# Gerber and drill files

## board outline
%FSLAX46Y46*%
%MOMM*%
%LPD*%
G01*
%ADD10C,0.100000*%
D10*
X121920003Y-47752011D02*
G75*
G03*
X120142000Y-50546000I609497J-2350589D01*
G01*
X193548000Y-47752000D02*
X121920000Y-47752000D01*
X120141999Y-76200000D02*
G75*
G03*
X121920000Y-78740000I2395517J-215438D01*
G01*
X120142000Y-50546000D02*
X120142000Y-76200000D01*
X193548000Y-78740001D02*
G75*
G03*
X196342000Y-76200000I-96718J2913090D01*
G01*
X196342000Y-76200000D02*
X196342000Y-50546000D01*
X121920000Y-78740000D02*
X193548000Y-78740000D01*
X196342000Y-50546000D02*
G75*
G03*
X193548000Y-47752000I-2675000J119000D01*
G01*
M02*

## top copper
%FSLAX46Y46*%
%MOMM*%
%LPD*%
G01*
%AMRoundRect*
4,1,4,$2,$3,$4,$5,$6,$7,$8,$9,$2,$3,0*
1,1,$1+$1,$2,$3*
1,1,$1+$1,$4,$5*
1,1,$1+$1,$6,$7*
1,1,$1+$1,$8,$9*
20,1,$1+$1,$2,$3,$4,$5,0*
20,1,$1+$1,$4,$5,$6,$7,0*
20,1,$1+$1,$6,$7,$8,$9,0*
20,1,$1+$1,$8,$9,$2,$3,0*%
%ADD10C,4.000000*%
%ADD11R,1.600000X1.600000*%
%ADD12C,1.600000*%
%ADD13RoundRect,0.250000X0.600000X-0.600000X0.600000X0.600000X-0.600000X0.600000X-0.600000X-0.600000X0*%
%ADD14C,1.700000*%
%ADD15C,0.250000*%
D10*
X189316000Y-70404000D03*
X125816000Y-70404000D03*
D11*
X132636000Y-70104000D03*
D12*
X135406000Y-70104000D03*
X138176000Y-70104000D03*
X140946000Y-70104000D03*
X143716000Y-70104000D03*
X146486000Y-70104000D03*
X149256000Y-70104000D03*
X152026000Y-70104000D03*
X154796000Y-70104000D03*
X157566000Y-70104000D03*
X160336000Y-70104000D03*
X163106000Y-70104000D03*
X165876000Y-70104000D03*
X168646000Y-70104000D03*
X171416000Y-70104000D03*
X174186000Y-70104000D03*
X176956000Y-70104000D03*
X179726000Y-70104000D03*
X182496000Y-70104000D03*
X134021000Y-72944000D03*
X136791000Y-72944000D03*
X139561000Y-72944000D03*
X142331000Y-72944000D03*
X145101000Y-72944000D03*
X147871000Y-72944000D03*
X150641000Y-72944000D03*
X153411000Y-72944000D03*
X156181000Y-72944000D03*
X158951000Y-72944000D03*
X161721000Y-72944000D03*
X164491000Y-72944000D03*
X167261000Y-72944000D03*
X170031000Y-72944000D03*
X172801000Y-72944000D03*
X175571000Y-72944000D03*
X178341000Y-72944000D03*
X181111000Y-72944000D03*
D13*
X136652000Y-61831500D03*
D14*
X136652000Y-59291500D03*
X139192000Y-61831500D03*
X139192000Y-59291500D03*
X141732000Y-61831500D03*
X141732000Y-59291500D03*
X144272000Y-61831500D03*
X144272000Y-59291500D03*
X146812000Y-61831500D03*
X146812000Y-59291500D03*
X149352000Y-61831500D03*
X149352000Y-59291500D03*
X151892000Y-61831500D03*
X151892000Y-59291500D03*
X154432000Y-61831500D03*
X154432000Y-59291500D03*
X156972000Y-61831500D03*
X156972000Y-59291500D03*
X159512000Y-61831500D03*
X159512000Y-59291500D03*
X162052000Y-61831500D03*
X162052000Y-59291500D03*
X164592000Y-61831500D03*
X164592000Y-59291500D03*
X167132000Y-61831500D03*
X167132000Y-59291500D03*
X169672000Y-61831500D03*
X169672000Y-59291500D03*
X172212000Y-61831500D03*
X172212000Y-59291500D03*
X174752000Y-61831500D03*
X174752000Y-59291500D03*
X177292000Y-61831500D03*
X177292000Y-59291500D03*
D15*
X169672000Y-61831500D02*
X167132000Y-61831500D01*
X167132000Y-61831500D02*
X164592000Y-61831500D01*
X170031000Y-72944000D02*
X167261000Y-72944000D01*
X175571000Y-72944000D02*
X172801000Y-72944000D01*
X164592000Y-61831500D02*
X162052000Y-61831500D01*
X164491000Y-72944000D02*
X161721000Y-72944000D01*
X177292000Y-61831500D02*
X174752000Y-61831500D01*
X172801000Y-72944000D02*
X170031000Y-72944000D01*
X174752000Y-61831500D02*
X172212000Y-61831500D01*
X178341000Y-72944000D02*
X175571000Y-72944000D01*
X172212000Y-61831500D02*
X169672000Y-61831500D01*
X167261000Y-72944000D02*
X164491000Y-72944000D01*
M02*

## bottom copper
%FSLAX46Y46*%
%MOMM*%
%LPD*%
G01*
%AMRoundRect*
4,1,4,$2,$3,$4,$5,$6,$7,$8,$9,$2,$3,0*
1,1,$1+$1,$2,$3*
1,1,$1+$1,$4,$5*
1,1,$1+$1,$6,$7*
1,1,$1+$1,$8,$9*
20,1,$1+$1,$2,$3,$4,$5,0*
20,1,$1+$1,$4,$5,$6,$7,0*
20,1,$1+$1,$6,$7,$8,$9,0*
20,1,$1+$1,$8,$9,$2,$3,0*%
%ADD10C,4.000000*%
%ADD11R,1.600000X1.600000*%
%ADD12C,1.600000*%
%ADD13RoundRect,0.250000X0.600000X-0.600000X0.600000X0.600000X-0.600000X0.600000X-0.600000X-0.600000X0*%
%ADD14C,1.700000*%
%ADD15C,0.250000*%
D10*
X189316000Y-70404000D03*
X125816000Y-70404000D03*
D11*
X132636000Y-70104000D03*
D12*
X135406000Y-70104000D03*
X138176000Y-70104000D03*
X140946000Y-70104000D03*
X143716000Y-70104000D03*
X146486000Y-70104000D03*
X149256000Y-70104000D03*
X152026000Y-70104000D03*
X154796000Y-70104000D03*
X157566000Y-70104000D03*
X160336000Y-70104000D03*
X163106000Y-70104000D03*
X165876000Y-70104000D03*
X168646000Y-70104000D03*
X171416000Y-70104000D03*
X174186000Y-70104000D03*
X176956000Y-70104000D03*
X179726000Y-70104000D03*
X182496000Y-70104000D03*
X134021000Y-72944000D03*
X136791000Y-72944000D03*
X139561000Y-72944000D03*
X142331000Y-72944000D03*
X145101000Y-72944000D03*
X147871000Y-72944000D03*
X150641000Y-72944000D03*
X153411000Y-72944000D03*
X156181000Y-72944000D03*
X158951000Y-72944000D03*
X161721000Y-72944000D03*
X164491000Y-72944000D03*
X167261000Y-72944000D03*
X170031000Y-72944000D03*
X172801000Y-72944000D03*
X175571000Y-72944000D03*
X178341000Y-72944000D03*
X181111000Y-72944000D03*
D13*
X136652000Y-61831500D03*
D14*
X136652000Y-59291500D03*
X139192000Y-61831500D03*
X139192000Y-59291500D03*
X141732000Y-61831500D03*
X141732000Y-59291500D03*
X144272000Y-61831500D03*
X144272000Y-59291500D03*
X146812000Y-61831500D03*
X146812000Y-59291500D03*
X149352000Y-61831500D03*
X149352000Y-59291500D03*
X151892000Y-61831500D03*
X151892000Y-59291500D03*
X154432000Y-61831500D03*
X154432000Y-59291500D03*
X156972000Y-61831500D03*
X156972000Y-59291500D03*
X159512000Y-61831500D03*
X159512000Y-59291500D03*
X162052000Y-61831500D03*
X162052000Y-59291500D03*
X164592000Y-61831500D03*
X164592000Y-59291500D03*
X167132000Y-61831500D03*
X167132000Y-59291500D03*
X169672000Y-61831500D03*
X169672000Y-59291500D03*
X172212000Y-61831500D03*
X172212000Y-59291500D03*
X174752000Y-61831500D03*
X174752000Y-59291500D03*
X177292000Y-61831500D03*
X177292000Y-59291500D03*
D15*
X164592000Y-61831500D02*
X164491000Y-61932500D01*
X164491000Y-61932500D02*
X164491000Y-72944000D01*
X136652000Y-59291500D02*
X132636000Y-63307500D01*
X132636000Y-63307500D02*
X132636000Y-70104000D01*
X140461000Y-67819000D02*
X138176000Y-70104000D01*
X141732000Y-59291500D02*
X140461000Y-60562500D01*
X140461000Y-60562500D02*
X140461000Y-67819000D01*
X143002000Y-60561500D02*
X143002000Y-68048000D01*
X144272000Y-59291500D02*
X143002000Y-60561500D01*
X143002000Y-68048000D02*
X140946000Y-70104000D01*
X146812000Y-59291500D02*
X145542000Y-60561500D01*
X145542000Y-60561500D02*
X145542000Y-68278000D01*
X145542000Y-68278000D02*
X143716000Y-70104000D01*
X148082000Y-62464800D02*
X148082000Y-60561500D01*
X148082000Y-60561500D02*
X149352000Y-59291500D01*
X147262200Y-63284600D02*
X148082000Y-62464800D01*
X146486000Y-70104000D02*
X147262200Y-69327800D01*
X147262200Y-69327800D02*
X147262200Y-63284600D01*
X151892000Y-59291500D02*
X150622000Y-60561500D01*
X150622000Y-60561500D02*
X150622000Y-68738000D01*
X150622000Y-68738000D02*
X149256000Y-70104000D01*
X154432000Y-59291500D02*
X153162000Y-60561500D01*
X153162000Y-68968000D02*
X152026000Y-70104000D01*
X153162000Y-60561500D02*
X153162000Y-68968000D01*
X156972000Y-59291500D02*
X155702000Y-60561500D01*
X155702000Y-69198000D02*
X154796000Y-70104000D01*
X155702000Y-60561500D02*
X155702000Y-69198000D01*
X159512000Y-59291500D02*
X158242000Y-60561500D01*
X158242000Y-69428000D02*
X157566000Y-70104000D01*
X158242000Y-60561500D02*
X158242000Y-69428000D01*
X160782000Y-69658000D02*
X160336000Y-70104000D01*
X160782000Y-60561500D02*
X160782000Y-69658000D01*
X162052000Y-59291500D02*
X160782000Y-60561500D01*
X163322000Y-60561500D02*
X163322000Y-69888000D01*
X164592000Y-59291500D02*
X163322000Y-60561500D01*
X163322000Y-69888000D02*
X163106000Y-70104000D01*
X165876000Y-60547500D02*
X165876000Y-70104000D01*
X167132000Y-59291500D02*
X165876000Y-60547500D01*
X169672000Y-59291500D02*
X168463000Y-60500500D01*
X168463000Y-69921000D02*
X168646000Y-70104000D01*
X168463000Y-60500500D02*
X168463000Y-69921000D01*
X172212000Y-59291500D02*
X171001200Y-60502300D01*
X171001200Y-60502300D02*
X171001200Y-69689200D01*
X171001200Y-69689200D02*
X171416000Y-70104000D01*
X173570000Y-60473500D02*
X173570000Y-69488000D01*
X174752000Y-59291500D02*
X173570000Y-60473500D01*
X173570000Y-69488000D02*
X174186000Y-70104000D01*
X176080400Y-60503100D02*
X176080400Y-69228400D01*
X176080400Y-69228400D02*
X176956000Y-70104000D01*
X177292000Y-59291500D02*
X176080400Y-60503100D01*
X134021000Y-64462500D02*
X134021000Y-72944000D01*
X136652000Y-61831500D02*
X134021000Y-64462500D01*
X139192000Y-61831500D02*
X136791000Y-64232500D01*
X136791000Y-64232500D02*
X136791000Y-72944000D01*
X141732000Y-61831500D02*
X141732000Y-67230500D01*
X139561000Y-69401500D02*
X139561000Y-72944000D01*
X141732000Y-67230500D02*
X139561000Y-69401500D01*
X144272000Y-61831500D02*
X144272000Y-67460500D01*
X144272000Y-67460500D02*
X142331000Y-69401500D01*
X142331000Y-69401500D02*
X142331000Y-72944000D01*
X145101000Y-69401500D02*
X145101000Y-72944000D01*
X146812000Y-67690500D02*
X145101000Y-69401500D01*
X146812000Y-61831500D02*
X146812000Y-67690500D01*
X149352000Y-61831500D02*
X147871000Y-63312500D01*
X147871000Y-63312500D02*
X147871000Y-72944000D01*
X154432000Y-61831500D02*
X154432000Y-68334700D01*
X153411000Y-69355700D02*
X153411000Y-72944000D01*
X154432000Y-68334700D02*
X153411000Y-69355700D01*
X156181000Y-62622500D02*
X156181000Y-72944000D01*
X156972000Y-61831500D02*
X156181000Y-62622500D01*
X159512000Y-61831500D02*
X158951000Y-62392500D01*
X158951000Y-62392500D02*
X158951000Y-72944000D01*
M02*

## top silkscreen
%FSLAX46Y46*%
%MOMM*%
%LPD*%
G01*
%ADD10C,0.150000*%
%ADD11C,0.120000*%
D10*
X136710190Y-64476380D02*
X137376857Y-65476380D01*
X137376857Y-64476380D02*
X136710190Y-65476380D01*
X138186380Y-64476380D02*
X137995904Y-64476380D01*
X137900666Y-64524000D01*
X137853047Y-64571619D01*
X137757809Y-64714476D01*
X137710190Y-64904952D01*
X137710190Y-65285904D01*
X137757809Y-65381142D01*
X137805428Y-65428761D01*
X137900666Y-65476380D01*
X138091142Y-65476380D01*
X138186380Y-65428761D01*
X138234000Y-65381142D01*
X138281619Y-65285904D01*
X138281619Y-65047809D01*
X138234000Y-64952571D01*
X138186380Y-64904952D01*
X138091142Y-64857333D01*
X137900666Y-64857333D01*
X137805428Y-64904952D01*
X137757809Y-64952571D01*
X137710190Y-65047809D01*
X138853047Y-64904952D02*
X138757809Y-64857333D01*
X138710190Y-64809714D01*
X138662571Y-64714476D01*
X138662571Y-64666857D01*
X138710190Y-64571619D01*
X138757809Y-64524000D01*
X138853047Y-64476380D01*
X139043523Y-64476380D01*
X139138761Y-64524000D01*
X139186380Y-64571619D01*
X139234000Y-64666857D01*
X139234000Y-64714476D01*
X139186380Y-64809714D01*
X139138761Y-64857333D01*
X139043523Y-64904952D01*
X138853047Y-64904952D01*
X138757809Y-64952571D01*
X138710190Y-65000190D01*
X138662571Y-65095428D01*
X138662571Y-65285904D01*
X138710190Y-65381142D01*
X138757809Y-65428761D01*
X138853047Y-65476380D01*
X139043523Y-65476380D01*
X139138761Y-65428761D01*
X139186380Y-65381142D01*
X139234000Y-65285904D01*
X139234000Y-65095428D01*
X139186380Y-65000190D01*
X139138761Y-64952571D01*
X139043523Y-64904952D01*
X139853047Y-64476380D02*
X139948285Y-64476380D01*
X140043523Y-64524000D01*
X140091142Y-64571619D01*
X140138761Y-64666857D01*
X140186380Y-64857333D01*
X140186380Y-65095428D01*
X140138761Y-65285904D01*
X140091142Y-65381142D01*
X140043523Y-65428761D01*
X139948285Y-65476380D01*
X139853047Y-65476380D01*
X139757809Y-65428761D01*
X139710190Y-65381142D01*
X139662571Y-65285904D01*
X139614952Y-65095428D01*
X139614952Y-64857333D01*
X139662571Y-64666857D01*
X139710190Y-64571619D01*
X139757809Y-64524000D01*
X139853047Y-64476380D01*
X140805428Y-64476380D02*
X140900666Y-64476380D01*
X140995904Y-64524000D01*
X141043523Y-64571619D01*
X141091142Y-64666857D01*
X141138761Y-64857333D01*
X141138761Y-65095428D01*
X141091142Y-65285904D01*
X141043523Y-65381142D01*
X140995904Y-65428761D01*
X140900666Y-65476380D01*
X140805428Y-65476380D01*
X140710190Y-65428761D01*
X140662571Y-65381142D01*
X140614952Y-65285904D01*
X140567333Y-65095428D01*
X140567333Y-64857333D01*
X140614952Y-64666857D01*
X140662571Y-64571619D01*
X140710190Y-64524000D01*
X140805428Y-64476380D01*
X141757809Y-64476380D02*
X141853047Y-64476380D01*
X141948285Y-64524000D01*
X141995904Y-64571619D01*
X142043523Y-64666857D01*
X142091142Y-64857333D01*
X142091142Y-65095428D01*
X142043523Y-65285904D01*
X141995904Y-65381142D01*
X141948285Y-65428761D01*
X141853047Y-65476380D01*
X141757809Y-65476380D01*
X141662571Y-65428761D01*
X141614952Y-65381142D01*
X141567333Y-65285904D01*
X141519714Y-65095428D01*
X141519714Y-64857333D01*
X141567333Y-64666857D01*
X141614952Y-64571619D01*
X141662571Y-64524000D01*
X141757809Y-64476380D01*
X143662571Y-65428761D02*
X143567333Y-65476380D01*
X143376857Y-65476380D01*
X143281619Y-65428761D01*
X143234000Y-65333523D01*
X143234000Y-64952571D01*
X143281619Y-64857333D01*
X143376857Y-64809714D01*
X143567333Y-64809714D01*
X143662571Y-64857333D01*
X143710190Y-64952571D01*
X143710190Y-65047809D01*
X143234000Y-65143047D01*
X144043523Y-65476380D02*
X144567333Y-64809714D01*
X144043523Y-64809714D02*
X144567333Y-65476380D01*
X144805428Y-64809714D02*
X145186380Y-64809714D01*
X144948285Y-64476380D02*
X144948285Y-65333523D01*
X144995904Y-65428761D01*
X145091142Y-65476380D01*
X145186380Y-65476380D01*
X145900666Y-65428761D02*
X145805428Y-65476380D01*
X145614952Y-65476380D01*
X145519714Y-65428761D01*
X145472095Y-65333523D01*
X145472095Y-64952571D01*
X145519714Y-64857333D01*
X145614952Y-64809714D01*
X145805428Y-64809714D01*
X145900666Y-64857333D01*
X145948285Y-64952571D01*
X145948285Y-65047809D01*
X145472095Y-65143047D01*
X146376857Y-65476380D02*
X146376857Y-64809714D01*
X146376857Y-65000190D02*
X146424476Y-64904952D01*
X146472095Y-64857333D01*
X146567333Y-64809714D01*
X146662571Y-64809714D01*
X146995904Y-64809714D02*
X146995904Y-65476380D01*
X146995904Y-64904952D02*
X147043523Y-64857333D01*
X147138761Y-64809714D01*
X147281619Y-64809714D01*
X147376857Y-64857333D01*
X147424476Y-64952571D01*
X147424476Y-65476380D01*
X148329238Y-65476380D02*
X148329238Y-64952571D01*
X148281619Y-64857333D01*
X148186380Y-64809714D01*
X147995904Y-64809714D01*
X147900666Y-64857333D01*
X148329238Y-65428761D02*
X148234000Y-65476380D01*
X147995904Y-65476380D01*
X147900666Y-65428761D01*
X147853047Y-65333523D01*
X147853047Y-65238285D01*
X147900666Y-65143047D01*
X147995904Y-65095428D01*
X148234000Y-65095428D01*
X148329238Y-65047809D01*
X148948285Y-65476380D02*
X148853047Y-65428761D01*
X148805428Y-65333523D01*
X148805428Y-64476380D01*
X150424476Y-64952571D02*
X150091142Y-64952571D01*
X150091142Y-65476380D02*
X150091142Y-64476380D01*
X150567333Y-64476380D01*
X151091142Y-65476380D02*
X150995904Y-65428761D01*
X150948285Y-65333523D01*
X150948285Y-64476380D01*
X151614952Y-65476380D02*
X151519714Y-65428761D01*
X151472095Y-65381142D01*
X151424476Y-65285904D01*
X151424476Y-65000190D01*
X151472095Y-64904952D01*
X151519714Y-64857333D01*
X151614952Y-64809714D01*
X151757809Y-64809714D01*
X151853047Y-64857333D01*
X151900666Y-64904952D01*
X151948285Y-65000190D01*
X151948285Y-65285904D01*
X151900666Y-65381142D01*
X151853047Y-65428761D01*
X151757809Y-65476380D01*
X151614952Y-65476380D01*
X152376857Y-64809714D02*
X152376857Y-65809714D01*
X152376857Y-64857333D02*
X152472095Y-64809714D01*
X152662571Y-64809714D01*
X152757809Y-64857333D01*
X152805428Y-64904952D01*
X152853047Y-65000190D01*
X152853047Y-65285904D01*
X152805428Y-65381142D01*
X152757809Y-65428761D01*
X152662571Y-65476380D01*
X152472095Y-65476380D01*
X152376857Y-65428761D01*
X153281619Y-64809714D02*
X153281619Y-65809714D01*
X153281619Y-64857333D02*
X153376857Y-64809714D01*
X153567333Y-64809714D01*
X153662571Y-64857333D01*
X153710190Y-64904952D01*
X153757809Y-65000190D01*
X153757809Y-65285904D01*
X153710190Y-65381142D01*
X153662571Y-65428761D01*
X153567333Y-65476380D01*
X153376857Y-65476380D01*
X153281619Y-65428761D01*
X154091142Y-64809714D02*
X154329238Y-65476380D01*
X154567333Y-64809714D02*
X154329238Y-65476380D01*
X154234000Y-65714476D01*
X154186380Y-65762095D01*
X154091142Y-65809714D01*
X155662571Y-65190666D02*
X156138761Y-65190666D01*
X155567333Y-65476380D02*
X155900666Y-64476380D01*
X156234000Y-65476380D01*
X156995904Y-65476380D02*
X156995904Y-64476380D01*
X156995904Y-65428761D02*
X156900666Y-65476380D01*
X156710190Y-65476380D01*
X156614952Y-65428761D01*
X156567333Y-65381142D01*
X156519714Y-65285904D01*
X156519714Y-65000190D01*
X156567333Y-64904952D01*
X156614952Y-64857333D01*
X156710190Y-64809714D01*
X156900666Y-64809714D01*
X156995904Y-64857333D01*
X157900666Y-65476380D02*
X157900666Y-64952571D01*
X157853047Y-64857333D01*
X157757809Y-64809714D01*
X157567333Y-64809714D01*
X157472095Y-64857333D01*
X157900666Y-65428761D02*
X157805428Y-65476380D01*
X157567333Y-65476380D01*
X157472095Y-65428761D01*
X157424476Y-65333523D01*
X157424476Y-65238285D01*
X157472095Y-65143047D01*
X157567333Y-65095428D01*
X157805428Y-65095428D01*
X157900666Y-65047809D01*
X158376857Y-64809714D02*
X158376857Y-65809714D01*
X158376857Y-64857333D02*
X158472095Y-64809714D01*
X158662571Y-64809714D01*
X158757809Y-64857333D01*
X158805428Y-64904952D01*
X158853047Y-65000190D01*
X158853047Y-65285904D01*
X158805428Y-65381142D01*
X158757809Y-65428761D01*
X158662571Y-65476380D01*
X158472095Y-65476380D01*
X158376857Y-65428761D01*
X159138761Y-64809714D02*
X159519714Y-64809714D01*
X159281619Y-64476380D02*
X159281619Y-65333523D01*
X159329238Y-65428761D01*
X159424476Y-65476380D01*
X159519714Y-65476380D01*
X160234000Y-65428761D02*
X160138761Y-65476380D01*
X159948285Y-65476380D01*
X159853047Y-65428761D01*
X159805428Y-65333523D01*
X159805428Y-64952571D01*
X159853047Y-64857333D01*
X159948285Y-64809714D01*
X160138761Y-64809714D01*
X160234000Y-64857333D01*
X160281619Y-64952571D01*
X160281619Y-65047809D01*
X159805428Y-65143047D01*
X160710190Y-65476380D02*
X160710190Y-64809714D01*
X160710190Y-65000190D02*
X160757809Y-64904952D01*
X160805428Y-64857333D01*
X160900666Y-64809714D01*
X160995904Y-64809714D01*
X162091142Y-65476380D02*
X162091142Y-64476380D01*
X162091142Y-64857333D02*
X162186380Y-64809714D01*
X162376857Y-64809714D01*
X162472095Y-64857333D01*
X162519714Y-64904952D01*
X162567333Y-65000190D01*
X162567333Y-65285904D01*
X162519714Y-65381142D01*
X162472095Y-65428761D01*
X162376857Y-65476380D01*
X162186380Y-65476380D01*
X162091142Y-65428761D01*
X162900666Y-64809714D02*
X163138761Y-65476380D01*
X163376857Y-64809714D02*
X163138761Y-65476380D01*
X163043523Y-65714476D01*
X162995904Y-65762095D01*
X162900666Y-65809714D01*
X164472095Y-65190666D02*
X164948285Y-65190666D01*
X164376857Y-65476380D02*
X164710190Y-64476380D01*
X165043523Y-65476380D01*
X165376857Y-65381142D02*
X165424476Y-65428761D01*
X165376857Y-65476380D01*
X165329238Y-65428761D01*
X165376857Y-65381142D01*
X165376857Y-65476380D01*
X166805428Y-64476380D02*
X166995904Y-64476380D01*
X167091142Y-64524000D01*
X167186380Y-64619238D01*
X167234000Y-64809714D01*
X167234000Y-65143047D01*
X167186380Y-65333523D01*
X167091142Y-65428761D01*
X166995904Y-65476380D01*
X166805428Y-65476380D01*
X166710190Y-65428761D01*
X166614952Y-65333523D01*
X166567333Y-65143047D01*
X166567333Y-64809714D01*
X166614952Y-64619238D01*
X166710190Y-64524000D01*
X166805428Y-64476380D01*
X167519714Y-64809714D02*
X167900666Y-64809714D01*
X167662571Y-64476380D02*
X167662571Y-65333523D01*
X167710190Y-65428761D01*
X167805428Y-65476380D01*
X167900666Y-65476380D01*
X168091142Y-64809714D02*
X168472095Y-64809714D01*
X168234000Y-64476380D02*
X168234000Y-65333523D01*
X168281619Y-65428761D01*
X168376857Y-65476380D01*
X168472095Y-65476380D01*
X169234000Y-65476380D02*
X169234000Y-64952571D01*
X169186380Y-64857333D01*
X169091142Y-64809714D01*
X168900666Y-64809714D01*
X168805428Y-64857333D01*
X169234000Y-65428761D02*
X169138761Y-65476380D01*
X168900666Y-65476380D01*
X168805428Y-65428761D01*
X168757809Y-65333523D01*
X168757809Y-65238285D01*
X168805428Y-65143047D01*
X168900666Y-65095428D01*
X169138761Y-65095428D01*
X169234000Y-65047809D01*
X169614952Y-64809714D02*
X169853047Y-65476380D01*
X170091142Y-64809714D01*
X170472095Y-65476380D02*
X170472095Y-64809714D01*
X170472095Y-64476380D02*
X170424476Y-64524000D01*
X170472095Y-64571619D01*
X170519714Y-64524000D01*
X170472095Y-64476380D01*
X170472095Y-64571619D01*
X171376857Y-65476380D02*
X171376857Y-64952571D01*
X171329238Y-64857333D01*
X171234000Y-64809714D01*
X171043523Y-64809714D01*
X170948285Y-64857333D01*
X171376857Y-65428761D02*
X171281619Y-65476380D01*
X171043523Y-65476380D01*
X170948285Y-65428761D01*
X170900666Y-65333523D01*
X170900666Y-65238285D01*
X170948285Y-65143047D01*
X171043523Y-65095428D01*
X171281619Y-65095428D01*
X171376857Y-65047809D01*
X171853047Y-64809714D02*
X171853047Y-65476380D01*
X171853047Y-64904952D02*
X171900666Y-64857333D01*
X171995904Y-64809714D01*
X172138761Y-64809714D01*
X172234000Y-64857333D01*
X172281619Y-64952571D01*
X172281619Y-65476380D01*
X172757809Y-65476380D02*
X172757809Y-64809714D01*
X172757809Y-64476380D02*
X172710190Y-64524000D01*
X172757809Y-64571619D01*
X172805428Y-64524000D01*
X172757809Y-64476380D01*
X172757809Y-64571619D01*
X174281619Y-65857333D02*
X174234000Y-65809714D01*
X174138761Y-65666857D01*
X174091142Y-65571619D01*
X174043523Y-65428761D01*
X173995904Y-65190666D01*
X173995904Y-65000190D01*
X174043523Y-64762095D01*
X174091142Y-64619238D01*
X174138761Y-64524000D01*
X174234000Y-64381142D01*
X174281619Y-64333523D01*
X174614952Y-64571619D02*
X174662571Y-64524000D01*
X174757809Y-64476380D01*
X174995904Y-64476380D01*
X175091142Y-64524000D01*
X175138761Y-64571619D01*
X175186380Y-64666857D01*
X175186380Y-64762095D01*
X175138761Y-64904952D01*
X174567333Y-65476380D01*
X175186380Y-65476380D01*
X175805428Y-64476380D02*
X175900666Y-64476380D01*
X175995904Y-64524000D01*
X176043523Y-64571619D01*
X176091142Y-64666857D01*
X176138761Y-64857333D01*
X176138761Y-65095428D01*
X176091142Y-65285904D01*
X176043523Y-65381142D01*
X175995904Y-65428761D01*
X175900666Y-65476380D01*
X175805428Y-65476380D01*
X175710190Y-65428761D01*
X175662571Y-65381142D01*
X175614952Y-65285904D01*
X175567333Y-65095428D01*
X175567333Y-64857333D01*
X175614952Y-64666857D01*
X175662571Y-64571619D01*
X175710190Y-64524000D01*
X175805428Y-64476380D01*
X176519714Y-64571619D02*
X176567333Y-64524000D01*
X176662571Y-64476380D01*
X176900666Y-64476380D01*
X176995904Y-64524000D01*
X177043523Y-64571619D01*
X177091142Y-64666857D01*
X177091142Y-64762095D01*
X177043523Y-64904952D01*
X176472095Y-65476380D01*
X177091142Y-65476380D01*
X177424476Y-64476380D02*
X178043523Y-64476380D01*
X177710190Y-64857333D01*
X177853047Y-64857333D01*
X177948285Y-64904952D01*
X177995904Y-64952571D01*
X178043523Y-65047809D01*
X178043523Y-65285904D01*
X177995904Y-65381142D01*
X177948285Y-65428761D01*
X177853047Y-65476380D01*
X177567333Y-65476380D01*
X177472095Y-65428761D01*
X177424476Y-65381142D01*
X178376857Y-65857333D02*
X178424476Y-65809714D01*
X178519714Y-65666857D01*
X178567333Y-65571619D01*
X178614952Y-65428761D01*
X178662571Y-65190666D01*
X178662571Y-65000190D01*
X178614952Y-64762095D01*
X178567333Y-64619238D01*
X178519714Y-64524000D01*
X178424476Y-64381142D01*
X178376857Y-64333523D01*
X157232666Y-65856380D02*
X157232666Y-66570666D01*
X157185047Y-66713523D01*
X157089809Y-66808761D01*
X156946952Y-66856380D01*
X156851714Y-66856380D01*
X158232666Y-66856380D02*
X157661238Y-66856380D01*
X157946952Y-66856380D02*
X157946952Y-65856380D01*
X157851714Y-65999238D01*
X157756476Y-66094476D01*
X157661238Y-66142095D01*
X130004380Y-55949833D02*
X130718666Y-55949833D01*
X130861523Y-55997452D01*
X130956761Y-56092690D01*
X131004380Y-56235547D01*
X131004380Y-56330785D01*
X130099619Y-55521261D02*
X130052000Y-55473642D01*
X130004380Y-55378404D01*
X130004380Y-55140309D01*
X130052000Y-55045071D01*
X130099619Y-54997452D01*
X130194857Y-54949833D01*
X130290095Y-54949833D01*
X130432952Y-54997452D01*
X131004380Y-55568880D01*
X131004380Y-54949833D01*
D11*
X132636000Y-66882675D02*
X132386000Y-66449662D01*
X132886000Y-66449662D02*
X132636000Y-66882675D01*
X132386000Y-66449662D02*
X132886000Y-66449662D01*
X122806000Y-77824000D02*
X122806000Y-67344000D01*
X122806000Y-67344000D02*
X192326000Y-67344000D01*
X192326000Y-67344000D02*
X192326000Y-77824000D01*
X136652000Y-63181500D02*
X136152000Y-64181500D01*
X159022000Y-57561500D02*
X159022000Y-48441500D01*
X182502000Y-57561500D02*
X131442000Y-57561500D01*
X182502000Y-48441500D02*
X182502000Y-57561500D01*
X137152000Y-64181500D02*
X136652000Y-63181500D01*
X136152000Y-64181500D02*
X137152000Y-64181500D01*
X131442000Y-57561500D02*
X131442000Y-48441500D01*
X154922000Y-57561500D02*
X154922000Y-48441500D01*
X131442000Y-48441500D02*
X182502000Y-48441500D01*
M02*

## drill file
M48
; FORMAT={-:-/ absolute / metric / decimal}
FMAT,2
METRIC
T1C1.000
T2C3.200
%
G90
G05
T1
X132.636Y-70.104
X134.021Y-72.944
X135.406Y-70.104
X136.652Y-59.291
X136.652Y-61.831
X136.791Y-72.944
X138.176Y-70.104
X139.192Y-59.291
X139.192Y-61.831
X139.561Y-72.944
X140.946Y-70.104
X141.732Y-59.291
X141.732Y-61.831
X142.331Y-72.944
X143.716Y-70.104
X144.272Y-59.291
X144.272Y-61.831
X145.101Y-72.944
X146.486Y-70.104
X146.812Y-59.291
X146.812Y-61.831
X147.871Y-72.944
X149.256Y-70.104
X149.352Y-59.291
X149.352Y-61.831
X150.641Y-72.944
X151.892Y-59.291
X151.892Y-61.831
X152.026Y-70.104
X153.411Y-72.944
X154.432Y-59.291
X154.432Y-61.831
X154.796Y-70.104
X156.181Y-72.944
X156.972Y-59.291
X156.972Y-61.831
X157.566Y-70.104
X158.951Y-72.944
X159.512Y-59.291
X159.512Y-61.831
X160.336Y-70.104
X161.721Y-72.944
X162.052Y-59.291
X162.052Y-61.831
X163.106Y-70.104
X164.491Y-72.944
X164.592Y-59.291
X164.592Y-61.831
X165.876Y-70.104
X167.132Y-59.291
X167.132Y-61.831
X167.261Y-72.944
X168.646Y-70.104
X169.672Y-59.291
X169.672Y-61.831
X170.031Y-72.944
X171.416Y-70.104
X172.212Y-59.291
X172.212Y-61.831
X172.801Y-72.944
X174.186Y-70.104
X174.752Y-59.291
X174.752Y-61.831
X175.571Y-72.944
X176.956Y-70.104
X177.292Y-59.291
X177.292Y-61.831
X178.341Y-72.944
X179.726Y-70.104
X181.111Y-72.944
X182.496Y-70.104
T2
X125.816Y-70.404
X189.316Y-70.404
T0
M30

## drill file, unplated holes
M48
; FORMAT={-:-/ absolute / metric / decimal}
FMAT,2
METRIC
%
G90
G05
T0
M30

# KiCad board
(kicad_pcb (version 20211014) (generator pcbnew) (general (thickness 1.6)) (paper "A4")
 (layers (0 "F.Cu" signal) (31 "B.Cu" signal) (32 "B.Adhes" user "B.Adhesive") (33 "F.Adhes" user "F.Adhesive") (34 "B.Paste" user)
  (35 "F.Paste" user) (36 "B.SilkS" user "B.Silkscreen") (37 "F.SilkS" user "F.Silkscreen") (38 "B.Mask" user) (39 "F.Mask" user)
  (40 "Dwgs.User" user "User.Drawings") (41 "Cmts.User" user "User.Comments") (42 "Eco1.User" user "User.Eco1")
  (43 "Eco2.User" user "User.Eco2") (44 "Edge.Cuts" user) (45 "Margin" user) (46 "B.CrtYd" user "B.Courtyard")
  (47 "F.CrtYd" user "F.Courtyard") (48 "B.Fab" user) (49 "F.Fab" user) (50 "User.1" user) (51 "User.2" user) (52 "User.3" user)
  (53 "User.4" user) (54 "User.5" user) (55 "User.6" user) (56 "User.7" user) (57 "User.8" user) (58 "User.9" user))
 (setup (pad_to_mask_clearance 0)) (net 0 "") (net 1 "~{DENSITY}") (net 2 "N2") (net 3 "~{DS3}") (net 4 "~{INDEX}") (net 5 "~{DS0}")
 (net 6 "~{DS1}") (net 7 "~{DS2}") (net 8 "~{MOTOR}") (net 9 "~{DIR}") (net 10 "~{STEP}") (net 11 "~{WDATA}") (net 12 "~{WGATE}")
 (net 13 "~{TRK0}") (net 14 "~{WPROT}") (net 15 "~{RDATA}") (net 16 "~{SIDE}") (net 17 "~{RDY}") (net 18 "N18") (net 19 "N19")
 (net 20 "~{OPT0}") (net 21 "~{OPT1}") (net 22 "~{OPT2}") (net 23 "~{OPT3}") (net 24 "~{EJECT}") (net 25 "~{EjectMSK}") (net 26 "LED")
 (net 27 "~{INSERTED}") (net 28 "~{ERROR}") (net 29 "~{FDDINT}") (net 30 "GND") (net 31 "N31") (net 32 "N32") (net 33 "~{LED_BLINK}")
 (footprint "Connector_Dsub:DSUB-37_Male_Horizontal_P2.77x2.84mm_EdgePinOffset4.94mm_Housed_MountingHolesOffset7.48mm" (layer "F.Cu")
  (at 132.636 70.104)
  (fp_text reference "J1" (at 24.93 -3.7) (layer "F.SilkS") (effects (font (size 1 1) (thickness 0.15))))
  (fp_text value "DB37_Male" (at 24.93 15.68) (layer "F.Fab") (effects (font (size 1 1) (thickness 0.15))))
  (fp_line (start 0 -3.221325) (end -0.25 -3.654338) (layer "F.SilkS") (width 0.12))
  (fp_line (start 0.25 -3.654338) (end 0 -3.221325) (layer "F.SilkS") (width 0.12))
  (fp_line (start -0.25 -3.654338) (end 0.25 -3.654338) (layer "F.SilkS") (width 0.12))
  (fp_line (start -9.83 7.72) (end -9.83 -2.76) (layer "F.SilkS") (width 0.12))
  (fp_line (start -9.83 -2.76) (end 59.69 -2.76) (layer "F.SilkS") (width 0.12))
  (fp_line (start 59.69 -2.76) (end 59.69 7.72) (layer "F.SilkS") (width 0.12))
  (pad "0" thru_hole circle (at 56.68 0.3) (size 4 4) (drill 3.2) (layers *.Cu *.Mask))
  (pad "0" thru_hole circle (at -6.82 0.3) (size 4 4) (drill 3.2) (layers *.Cu *.Mask))
  (pad "1" thru_hole rect (at 0 0) (size 1.6 1.6) (drill 1) (layers *.Cu *.Mask) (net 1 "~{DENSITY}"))
  (pad "2" thru_hole circle (at 2.77 0) (size 1.6 1.6) (drill 1) (layers *.Cu *.Mask) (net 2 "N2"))
  (pad "3" thru_hole circle (at 5.54 0) (size 1.6 1.6) (drill 1) (layers *.Cu *.Mask) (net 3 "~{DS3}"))
  (pad "4" thru_hole circle (at 8.31 0) (size 1.6 1.6) (drill 1) (layers *.Cu *.Mask) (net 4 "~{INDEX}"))
  (pad "5" thru_hole circle (at 11.08 0) (size 1.6 1.6) (drill 1) (layers *.Cu *.Mask) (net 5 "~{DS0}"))
  (pad "6" thru_hole circle (at 13.85 0) (size 1.6 1.6) (drill 1) (layers *.Cu *.Mask) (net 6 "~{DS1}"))
  (pad "7" thru_hole circle (at 16.62 0) (size 1.6 1.6) (drill 1) (layers *.Cu *.Mask) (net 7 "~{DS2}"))
  (pad "8" thru_hole circle (at 19.39 0) (size 1.6 1.6) (drill 1) (layers *.Cu *.Mask) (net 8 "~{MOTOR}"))
  (pad "9" thru_hole circle (at 22.16 0) (size 1.6 1.6) (drill 1) (layers *.Cu *.Mask) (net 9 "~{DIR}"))
  (pad "10" thru_hole circle (at 24.93 0) (size 1.6 1.6) (drill 1) (layers *.Cu *.Mask) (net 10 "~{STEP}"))
  (pad "11" thru_hole circle (at 27.7 0) (size 1.6 1.6) (drill 1) (layers *.Cu *.Mask) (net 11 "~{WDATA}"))
  (pad "12" thru_hole circle (at 30.47 0) (size 1.6 1.6) (drill 1) (layers *.Cu *.Mask) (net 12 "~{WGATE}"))
  (pad "13" thru_hole circle (at 33.24 0) (size 1.6 1.6) (drill 1) (layers *.Cu *.Mask) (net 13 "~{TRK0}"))
  (pad "14" thru_hole circle (at 36.01 0) (size 1.6 1.6) (drill 1) (layers *.Cu *.Mask) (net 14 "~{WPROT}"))
  (pad "15" thru_hole circle (at 38.78 0) (size 1.6 1.6) (drill 1) (layers *.Cu *.Mask) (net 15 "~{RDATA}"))
  (pad "16" thru_hole circle (at 41.55 0) (size 1.6 1.6) (drill 1) (layers *.Cu *.Mask) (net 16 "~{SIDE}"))
  (pad "17" thru_hole circle (at 44.32 0) (size 1.6 1.6) (drill 1) (layers *.Cu *.Mask) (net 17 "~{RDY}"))
  (pad "18" thru_hole circle (at 47.09 0) (size 1.6 1.6) (drill 1) (layers *.Cu *.Mask) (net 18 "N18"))
  (pad "19" thru_hole circle (at 49.86 0) (size 1.6 1.6) (drill 1) (layers *.Cu *.Mask) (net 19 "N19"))
  (pad "20" thru_hole circle (at 1.385 2.84) (size 1.6 1.6) (drill 1) (layers *.Cu *.Mask) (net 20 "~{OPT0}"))
  (pad "21" thru_hole circle (at 4.155 2.84) (size 1.6 1.6) (drill 1) (layers *.Cu *.Mask) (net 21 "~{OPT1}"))
  (pad "22" thru_hole circle (at 6.925 2.84) (size 1.6 1.6) (drill 1) (layers *.Cu *.Mask) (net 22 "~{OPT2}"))
  (pad "23" thru_hole circle (at 9.695 2.84) (size 1.6 1.6) (drill 1) (layers *.Cu *.Mask) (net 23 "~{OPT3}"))
  (pad "24" thru_hole circle (at 12.465 2.84) (size 1.6 1.6) (drill 1) (layers *.Cu *.Mask) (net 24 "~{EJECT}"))
  (pad "25" thru_hole circle (at 15.235 2.84) (size 1.6 1.6) (drill 1) (layers *.Cu *.Mask) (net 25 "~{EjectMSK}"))
  (pad "26" thru_hole circle (at 18.005 2.84) (size 1.6 1.6) (drill 1) (layers *.Cu *.Mask) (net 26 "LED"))
  (pad "27" thru_hole circle (at 20.775 2.84) (size 1.6 1.6) (drill 1) (layers *.Cu *.Mask) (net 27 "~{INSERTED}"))
  (pad "28" thru_hole circle (at 23.545 2.84) (size 1.6 1.6) (drill 1) (layers *.Cu *.Mask) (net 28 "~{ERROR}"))
  (pad "29" thru_hole circle (at 26.315 2.84) (size 1.6 1.6) (drill 1) (layers *.Cu *.Mask) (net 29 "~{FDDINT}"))
  (pad "30" thru_hole circle (at 29.085 2.84) (size 1.6 1.6) (drill 1) (layers *.Cu *.Mask) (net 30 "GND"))
  (pad "31" thru_hole circle (at 31.855 2.84) (size 1.6 1.6) (drill 1) (layers *.Cu *.Mask) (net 30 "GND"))
  (pad "32" thru_hole circle (at 34.625 2.84) (size 1.6 1.6) (drill 1) (layers *.Cu *.Mask) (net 30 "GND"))
  (pad "33" thru_hole circle (at 37.395 2.84) (size 1.6 1.6) (drill 1) (layers *.Cu *.Mask) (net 30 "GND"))
  (pad "34" thru_hole circle (at 40.165 2.84) (size 1.6 1.6) (drill 1) (layers *.Cu *.Mask) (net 30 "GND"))
  (pad "35" thru_hole circle (at 42.935 2.84) (size 1.6 1.6) (drill 1) (layers *.Cu *.Mask) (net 30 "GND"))
  (pad "36" thru_hole circle (at 45.705 2.84) (size 1.6 1.6) (drill 1) (layers *.Cu *.Mask) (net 30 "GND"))
  (pad "37" thru_hole circle (at 48.475 2.84) (size 1.6 1.6) (drill 1) (layers *.Cu *.Mask) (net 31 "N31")))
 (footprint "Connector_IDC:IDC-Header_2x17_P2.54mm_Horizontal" (layer "F.Cu") (at 136.652 61.8315 90)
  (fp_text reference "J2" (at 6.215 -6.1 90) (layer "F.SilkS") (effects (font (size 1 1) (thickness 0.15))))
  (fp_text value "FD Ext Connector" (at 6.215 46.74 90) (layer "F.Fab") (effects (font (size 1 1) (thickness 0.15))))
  (fp_line (start -1.35 0) (end -2.35 -0.5) (layer "F.SilkS") (width 0.12))
  (fp_line (start 4.27 22.37) (end 13.39 22.37) (layer "F.SilkS") (width 0.12))
  (fp_line (start 4.27 45.85) (end 4.27 -5.21) (layer "F.SilkS") (width 0.12))
  (fp_line (start 13.39 45.85) (end 4.27 45.85) (layer "F.SilkS") (width 0.12))
  (fp_line (start -2.35 0.5) (end -1.35 0) (layer "F.SilkS") (width 0.12))
  (fp_line (start -2.35 -0.5) (end -2.35 0.5) (layer "F.SilkS") (width 0.12))
  (fp_line (start 4.27 -5.21) (end 13.39 -5.21) (layer "F.SilkS") (width 0.12))
  (fp_line (start 4.27 18.27) (end 13.39 18.27) (layer "F.SilkS") (width 0.12))
  (fp_line (start 13.39 -5.21) (end 13.39 45.85) (layer "F.SilkS") (width 0.12))
  (pad "1" thru_hole roundrect (at 0 0 90) (size 1.7 1.7) (drill 1) (layers *.Cu *.Mask) (roundrect_rratio 0.147059) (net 20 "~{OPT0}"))
  (pad "2" thru_hole circle (at 2.54 0 90) (size 1.7 1.7) (drill 1) (layers *.Cu *.Mask) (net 1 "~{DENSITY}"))
  (pad "3" thru_hole circle (at 0 2.54 90) (size 1.7 1.7) (drill 1) (layers *.Cu *.Mask) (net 21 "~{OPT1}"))
  (pad "4" thru_hole circle (at 2.54 2.54 90) (size 1.7 1.7) (drill 1) (layers *.Cu *.Mask) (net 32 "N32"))
  (pad "5" thru_hole circle (at 0 5.08 90) (size 1.7 1.7) (drill 1) (layers *.Cu *.Mask) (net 22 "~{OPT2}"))
  (pad "6" thru_hole circle (at 2.54 5.08 90) (size 1.7 1.7) (drill 1) (layers *.Cu *.Mask) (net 3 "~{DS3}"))
  (pad "7" thru_hole circle (at 0 7.62 90) (size 1.7 1.7) (drill 1) (layers *.Cu *.Mask) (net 23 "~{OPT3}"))
  (pad "8" thru_hole circle (at 2.54 7.62 90) (size 1.7 1.7) (drill 1) (layers *.Cu *.Mask) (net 4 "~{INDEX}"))
  (pad "9" thru_hole circle (at 0 10.16 90) (size 1.7 1.7) (drill 1) (layers *.Cu *.Mask) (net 24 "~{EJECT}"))
  (pad "10" thru_hole circle (at 2.54 10.16 90) (size 1.7 1.7) (drill 1) (layers *.Cu *.Mask) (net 5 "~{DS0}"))
  (pad "11" thru_hole circle (at 0 12.7 90) (size 1.7 1.7) (drill 1) (layers *.Cu *.Mask) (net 25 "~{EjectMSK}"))
  (pad "12" thru_hole circle (at 2.54 12.7 90) (size 1.7 1.7) (drill 1) (layers *.Cu *.Mask) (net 6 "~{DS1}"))
  (pad "13" thru_hole circle (at 0 15.24 90) (size 1.7 1.7) (drill 1) (layers *.Cu *.Mask) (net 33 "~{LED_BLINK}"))
  (pad "14" thru_hole circle (at 2.54 15.24 90) (size 1.7 1.7) (drill 1) (layers *.Cu *.Mask) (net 7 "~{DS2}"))
  (pad "15" thru_hole circle (at 0 17.78 90) (size 1.7 1.7) (drill 1) (layers *.Cu *.Mask) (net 27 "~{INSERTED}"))
  (pad "16" thru_hole circle (at 2.54 17.78 90) (size 1.7 1.7) (drill 1) (layers *.Cu *.Mask) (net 8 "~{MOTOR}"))
  (pad "17" thru_hole circle (at 0 20.32 90) (size 1.7 1.7) (drill 1) (layers *.Cu *.Mask) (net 28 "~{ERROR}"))
  (pad "18" thru_hole circle (at 2.54 20.32 90) (size 1.7 1.7) (drill 1) (layers *.Cu *.Mask) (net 9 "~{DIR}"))
  (pad "19" thru_hole circle (at 0 22.86 90) (size 1.7 1.7) (drill 1) (layers *.Cu *.Mask) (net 29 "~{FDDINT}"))
  (pad "20" thru_hole circle (at 2.54 22.86 90) (size 1.7 1.7) (drill 1) (layers *.Cu *.Mask) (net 10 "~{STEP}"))
  (pad "21" thru_hole circle (at 0 25.4 90) (size 1.7 1.7) (drill 1) (layers *.Cu *.Mask) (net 30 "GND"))
  (pad "22" thru_hole circle (at 2.54 25.4 90) (size 1.7 1.7) (drill 1) (layers *.Cu *.Mask) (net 11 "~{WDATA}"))
  (pad "23" thru_hole circle (at 0 27.94 90) (size 1.7 1.7) (drill 1) (layers *.Cu *.Mask) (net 30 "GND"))
  (pad "24" thru_hole circle (at 2.54 27.94 90) (size 1.7 1.7) (drill 1) (layers *.Cu *.Mask) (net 12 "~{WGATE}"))
  (pad "25" thru_hole circle (at 0 30.48 90) (size 1.7 1.7) (drill 1) (layers *.Cu *.Mask) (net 30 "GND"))
  (pad "26" thru_hole circle (at 2.54 30.48 90) (size 1.7 1.7) (drill 1) (layers *.Cu *.Mask) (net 13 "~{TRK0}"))
  (pad "27" thru_hole circle (at 0 33.02 90) (size 1.7 1.7) (drill 1) (layers *.Cu *.Mask) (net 30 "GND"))
  (pad "28" thru_hole circle (at 2.54 33.02 90) (size 1.7 1.7) (drill 1) (layers *.Cu *.Mask) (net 14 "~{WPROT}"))
  (pad "29" thru_hole circle (at 0 35.56 90) (size 1.7 1.7) (drill 1) (layers *.Cu *.Mask) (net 30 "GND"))
  (pad "30" thru_hole circle (at 2.54 35.56 90) (size 1.7 1.7) (drill 1) (layers *.Cu *.Mask) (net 15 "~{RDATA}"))
  (pad "31" thru_hole circle (at 0 38.1 90) (size 1.7 1.7) (drill 1) (layers *.Cu *.Mask) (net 30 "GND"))
  (pad "32" thru_hole circle (at 2.54 38.1 90) (size 1.7 1.7) (drill 1) (layers *.Cu *.Mask) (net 16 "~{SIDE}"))
  (pad "33" thru_hole circle (at 0 40.64 90) (size 1.7 1.7) (drill 1) (layers *.Cu *.Mask) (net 30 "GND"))
  (pad "34" thru_hole circle (at 2.54 40.64 90) (size 1.7 1.7) (drill 1) (layers *.Cu *.Mask) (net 17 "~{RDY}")))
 (gr_arc (start 120.142 50.546) (mid 120.480812 48.79888) (end 121.92 47.752) (layer "Edge.Cuts") (width 0.1))
 (gr_line (start 193.548 47.752) (end 121.92 47.752) (layer "Edge.Cuts") (width 0.1))
 (gr_arc (start 121.92 78.74) (mid 120.567112 77.794721) (end 120.142 76.2) (layer "Edge.Cuts") (width 0.1))
 (gr_line (start 120.142 50.546) (end 120.142 76.2) (layer "Edge.Cuts") (width 0.1))
 (gr_arc (start 196.342 76.2) (mid 195.411918 77.98361) (end 193.548 78.74) (layer "Edge.Cuts") (width 0.1))
 (gr_line (start 196.342 76.2) (end 196.342 50.546) (layer "Edge.Cuts") (width 0.1))
 (gr_line (start 121.92 78.74) (end 193.548 78.74) (layer "Edge.Cuts") (width 0.1))
 (gr_arc (start 193.548 47.752) (mid 195.560386 48.533614) (end 196.342 50.546) (layer "Edge.Cuts") (width 0.1))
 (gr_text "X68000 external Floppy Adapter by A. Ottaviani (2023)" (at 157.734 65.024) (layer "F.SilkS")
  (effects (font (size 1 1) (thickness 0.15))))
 (segment (start 169.672 61.8315) (end 167.132 61.8315) (width 0.25) (layer "F.Cu") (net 30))
 (segment (start 167.132 61.8315) (end 164.592 61.8315) (width 0.25) (layer "F.Cu") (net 30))
 (segment (start 170.031 72.944) (end 167.261 72.944) (width 0.25) (layer "F.Cu") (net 30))
 (segment (start 175.571 72.944) (end 172.801 72.944) (width 0.25) (layer "F.Cu") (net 30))
 (segment (start 164.592 61.8315) (end 162.052 61.8315) (width 0.25) (layer "F.Cu") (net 30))
 (segment (start 164.491 72.944) (end 161.721 72.944) (width 0.25) (layer "F.Cu") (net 30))
 (segment (start 177.292 61.8315) (end 174.752 61.8315) (width 0.25) (layer "F.Cu") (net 30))
 (segment (start 172.801 72.944) (end 170.031 72.944) (width 0.25) (layer "F.Cu") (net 30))
 (segment (start 174.752 61.8315) (end 172.212 61.8315) (width 0.25) (layer "F.Cu") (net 30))
 (segment (start 178.341 72.944) (end 175.571 72.944) (width 0.25) (layer "F.Cu") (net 30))
 (segment (start 172.212 61.8315) (end 169.672 61.8315) (width 0.25) (layer "F.Cu") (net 30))
 (segment (start 167.261 72.944) (end 164.491 72.944) (width 0.25) (layer "F.Cu") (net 30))
 (segment (start 164.592 61.8315) (end 164.491 61.9325) (width 0.25) (layer "B.Cu") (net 30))
 (segment (start 164.491 61.9325) (end 164.491 72.944) (width 0.25) (layer "B.Cu") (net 30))
 (segment (start 136.652 59.2915) (end 132.636 63.3075) (width 0.25) (layer "B.Cu") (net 1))
 (segment (start 132.636 63.3075) (end 132.636 70.104) (width 0.25) (layer "B.Cu") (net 1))
 (segment (start 140.461 67.819) (end 138.176 70.104) (width 0.25) (layer "B.Cu") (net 3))
 (segment (start 141.732 59.2915) (end 140.461 60.5625) (width 0.25) (layer "B.Cu") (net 3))
 (segment (start 140.461 60.5625) (end 140.461 67.819) (width 0.25) (layer "B.Cu") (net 3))
 (segment (start 143.002 60.5615) (end 143.002 68.048) (width 0.25) (layer "B.Cu") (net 4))
 (segment (start 144.272 59.2915) (end 143.002 60.5615) (width 0.25) (layer "B.Cu") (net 4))
 (segment (start 143.002 68.048) (end 140.946 70.104) (width 0.25) (layer "B.Cu") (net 4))
 (segment (start 146.812 59.2915) (end 145.542 60.5615) (width 0.25) (layer "B.Cu") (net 5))
 (segment (start 145.542 60.5615) (end 145.542 68.278) (width 0.25) (layer "B.Cu") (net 5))
 (segment (start 145.542 68.278) (end 143.716 70.104) (width 0.25) (layer "B.Cu") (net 5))
 (segment (start 148.082 62.4648) (end 148.082 60.5615) (width 0.25) (layer "B.Cu") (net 6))
 (segment (start 148.082 60.5615) (end 149.352 59.2915) (width 0.25) (layer "B.Cu") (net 6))
 (segment (start 147.2622 63.2846) (end 148.082 62.4648) (width 0.25) (layer "B.Cu") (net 6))
 (segment (start 146.486 70.104) (end 147.2622 69.3278) (width 0.25) (layer "B.Cu") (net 6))
 (segment (start 147.2622 69.3278) (end 147.2622 63.2846) (width 0.25) (layer "B.Cu") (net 6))
 (segment (start 151.892 59.2915) (end 150.622 60.5615) (width 0.25) (layer "B.Cu") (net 7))
 (segment (start 150.622 60.5615) (end 150.622 68.738) (width 0.25) (layer "B.Cu") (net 7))
 (segment (start 150.622 68.738) (end 149.256 70.104) (width 0.25) (layer "B.Cu") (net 7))
 (segment (start 154.432 59.2915) (end 153.162 60.5615) (width 0.25) (layer "B.Cu") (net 8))
 (segment (start 153.162 68.968) (end 152.026 70.104) (width 0.25) (layer "B.Cu") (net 8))
 (segment (start 153.162 60.5615) (end 153.162 68.968) (width 0.25) (layer "B.Cu") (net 8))
 (segment (start 156.972 59.2915) (end 155.702 60.5615) (width 0.25) (layer "B.Cu") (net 9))
 (segment (start 155.702 69.198) (end 154.796 70.104) (width 0.25) (layer "B.Cu") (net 9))
 (segment (start 155.702 60.5615) (end 155.702 69.198) (width 0.25) (layer "B.Cu") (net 9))
 (segment (start 159.512 59.2915) (end 158.242 60.5615) (width 0.25) (layer "B.Cu") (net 10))
 (segment (start 158.242 69.428) (end 157.566 70.104) (width 0.25) (layer "B.Cu") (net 10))
 (segment (start 158.242 60.5615) (end 158.242 69.428) (width 0.25) (layer "B.Cu") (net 10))
 (segment (start 160.782 69.658) (end 160.336 70.104) (width 0.25) (layer "B.Cu") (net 11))
 (segment (start 160.782 60.5615) (end 160.782 69.658) (width 0.25) (layer "B.Cu") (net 11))
 (segment (start 162.052 59.2915) (end 160.782 60.5615) (width 0.25) (layer "B.Cu") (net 11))
 (segment (start 163.322 60.5615) (end 163.322 69.888) (width 0.25) (layer "B.Cu") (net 12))
 (segment (start 164.592 59.2915) (end 163.322 60.5615) (width 0.25) (layer "B.Cu") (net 12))
 (segment (start 163.322 69.888) (end 163.106 70.104) (width 0.25) (layer "B.Cu") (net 12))
 (segment (start 165.876 60.5475) (end 165.876 70.104) (width 0.25) (layer "B.Cu") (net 13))
 (segment (start 167.132 59.2915) (end 165.876 60.5475) (width 0.25) (layer "B.Cu") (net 13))
 (segment (start 169.672 59.2915) (end 168.463 60.5005) (width 0.25) (layer "B.Cu") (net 14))
 (segment (start 168.463 69.921) (end 168.646 70.104) (width 0.25) (layer "B.Cu") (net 14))
 (segment (start 168.463 60.5005) (end 168.463 69.921) (width 0.25) (layer "B.Cu") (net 14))
 (segment (start 172.212 59.2915) (end 171.0012 60.5023) (width 0.25) (layer "B.Cu") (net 15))
 (segment (start 171.0012 60.5023) (end 171.0012 69.6892) (width 0.25) (layer "B.Cu") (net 15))
 (segment (start 171.0012 69.6892) (end 171.416 70.104) (width 0.25) (layer "B.Cu") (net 15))
 (segment (start 173.57 60.4735) (end 173.57 69.488) (width 0.25) (layer "B.Cu") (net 16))
 (segment (start 174.752 59.2915) (end 173.57 60.4735) (width 0.25) (layer "B.Cu") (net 16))
 (segment (start 173.57 69.488) (end 174.186 70.104) (width 0.25) (layer "B.Cu") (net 16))
 (segment (start 176.0804 60.5031) (end 176.0804 69.2284) (width 0.25) (layer "B.Cu") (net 17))
 (segment (start 176.0804 69.2284) (end 176.956 70.104) (width 0.25) (layer "B.Cu") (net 17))
 (segment (start 177.292 59.2915) (end 176.0804 60.5031) (width 0.25) (layer "B.Cu") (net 17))
 (segment (start 134.021 64.4625) (end 134.021 72.944) (width 0.25) (layer "B.Cu") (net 20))
 (segment (start 136.652 61.8315) (end 134.021 64.4625) (width 0.25) (layer "B.Cu") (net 20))
 (segment (start 139.192 61.8315) (end 136.791 64.2325) (width 0.25) (layer "B.Cu") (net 21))
 (segment (start 136.791 64.2325) (end 136.791 72.944) (width 0.25) (layer "B.Cu") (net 21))
 (segment (start 141.732 61.8315) (end 141.732 67.2305) (width 0.25) (layer "B.Cu") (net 22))
 (segment (start 139.561 69.4015) (end 139.561 72.944) (width 0.25) (layer "B.Cu") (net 22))
 (segment (start 141.732 67.2305) (end 139.561 69.4015) (width 0.25) (layer "B.Cu") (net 22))
 (segment (start 144.272 61.8315) (end 144.272 67.4605) (width 0.25) (layer "B.Cu") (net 23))
 (segment (start 144.272 67.4605) (end 142.331 69.4015) (width 0.25) (layer "B.Cu") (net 23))
 (segment (start 142.331 69.4015) (end 142.331 72.944) (width 0.25) (layer "B.Cu") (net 23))
 (segment (start 145.101 69.4015) (end 145.101 72.944) (width 0.25) (layer "B.Cu") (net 24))
 (segment (start 146.812 67.6905) (end 145.101 69.4015) (width 0.25) (layer "B.Cu") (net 24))
 (segment (start 146.812 61.8315) (end 146.812 67.6905) (width 0.25) (layer "B.Cu") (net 24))
 (segment (start 149.352 61.8315) (end 147.871 63.3125) (width 0.25) (layer "B.Cu") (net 25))
 (segment (start 147.871 63.3125) (end 147.871 72.944) (width 0.25) (layer "B.Cu") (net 25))
 (segment (start 154.432 61.8315) (end 154.432 68.3347) (width 0.25) (layer "B.Cu") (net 27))
 (segment (start 153.411 69.3557) (end 153.411 72.944) (width 0.25) (layer "B.Cu") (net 27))
 (segment (start 154.432 68.3347) (end 153.411 69.3557) (width 0.25) (layer "B.Cu") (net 27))
 (segment (start 156.181 62.6225) (end 156.181 72.944) (width 0.25) (layer "B.Cu") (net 28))
 (segment (start 156.972 61.8315) (end 156.181 62.6225) (width 0.25) (layer "B.Cu") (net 28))
 (segment (start 159.512 61.8315) (end 158.951 62.3925) (width 0.25) (layer "B.Cu") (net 29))
 (segment (start 158.951 62.3925) (end 158.951 72.944) (width 0.25) (layer "B.Cu") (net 29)))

